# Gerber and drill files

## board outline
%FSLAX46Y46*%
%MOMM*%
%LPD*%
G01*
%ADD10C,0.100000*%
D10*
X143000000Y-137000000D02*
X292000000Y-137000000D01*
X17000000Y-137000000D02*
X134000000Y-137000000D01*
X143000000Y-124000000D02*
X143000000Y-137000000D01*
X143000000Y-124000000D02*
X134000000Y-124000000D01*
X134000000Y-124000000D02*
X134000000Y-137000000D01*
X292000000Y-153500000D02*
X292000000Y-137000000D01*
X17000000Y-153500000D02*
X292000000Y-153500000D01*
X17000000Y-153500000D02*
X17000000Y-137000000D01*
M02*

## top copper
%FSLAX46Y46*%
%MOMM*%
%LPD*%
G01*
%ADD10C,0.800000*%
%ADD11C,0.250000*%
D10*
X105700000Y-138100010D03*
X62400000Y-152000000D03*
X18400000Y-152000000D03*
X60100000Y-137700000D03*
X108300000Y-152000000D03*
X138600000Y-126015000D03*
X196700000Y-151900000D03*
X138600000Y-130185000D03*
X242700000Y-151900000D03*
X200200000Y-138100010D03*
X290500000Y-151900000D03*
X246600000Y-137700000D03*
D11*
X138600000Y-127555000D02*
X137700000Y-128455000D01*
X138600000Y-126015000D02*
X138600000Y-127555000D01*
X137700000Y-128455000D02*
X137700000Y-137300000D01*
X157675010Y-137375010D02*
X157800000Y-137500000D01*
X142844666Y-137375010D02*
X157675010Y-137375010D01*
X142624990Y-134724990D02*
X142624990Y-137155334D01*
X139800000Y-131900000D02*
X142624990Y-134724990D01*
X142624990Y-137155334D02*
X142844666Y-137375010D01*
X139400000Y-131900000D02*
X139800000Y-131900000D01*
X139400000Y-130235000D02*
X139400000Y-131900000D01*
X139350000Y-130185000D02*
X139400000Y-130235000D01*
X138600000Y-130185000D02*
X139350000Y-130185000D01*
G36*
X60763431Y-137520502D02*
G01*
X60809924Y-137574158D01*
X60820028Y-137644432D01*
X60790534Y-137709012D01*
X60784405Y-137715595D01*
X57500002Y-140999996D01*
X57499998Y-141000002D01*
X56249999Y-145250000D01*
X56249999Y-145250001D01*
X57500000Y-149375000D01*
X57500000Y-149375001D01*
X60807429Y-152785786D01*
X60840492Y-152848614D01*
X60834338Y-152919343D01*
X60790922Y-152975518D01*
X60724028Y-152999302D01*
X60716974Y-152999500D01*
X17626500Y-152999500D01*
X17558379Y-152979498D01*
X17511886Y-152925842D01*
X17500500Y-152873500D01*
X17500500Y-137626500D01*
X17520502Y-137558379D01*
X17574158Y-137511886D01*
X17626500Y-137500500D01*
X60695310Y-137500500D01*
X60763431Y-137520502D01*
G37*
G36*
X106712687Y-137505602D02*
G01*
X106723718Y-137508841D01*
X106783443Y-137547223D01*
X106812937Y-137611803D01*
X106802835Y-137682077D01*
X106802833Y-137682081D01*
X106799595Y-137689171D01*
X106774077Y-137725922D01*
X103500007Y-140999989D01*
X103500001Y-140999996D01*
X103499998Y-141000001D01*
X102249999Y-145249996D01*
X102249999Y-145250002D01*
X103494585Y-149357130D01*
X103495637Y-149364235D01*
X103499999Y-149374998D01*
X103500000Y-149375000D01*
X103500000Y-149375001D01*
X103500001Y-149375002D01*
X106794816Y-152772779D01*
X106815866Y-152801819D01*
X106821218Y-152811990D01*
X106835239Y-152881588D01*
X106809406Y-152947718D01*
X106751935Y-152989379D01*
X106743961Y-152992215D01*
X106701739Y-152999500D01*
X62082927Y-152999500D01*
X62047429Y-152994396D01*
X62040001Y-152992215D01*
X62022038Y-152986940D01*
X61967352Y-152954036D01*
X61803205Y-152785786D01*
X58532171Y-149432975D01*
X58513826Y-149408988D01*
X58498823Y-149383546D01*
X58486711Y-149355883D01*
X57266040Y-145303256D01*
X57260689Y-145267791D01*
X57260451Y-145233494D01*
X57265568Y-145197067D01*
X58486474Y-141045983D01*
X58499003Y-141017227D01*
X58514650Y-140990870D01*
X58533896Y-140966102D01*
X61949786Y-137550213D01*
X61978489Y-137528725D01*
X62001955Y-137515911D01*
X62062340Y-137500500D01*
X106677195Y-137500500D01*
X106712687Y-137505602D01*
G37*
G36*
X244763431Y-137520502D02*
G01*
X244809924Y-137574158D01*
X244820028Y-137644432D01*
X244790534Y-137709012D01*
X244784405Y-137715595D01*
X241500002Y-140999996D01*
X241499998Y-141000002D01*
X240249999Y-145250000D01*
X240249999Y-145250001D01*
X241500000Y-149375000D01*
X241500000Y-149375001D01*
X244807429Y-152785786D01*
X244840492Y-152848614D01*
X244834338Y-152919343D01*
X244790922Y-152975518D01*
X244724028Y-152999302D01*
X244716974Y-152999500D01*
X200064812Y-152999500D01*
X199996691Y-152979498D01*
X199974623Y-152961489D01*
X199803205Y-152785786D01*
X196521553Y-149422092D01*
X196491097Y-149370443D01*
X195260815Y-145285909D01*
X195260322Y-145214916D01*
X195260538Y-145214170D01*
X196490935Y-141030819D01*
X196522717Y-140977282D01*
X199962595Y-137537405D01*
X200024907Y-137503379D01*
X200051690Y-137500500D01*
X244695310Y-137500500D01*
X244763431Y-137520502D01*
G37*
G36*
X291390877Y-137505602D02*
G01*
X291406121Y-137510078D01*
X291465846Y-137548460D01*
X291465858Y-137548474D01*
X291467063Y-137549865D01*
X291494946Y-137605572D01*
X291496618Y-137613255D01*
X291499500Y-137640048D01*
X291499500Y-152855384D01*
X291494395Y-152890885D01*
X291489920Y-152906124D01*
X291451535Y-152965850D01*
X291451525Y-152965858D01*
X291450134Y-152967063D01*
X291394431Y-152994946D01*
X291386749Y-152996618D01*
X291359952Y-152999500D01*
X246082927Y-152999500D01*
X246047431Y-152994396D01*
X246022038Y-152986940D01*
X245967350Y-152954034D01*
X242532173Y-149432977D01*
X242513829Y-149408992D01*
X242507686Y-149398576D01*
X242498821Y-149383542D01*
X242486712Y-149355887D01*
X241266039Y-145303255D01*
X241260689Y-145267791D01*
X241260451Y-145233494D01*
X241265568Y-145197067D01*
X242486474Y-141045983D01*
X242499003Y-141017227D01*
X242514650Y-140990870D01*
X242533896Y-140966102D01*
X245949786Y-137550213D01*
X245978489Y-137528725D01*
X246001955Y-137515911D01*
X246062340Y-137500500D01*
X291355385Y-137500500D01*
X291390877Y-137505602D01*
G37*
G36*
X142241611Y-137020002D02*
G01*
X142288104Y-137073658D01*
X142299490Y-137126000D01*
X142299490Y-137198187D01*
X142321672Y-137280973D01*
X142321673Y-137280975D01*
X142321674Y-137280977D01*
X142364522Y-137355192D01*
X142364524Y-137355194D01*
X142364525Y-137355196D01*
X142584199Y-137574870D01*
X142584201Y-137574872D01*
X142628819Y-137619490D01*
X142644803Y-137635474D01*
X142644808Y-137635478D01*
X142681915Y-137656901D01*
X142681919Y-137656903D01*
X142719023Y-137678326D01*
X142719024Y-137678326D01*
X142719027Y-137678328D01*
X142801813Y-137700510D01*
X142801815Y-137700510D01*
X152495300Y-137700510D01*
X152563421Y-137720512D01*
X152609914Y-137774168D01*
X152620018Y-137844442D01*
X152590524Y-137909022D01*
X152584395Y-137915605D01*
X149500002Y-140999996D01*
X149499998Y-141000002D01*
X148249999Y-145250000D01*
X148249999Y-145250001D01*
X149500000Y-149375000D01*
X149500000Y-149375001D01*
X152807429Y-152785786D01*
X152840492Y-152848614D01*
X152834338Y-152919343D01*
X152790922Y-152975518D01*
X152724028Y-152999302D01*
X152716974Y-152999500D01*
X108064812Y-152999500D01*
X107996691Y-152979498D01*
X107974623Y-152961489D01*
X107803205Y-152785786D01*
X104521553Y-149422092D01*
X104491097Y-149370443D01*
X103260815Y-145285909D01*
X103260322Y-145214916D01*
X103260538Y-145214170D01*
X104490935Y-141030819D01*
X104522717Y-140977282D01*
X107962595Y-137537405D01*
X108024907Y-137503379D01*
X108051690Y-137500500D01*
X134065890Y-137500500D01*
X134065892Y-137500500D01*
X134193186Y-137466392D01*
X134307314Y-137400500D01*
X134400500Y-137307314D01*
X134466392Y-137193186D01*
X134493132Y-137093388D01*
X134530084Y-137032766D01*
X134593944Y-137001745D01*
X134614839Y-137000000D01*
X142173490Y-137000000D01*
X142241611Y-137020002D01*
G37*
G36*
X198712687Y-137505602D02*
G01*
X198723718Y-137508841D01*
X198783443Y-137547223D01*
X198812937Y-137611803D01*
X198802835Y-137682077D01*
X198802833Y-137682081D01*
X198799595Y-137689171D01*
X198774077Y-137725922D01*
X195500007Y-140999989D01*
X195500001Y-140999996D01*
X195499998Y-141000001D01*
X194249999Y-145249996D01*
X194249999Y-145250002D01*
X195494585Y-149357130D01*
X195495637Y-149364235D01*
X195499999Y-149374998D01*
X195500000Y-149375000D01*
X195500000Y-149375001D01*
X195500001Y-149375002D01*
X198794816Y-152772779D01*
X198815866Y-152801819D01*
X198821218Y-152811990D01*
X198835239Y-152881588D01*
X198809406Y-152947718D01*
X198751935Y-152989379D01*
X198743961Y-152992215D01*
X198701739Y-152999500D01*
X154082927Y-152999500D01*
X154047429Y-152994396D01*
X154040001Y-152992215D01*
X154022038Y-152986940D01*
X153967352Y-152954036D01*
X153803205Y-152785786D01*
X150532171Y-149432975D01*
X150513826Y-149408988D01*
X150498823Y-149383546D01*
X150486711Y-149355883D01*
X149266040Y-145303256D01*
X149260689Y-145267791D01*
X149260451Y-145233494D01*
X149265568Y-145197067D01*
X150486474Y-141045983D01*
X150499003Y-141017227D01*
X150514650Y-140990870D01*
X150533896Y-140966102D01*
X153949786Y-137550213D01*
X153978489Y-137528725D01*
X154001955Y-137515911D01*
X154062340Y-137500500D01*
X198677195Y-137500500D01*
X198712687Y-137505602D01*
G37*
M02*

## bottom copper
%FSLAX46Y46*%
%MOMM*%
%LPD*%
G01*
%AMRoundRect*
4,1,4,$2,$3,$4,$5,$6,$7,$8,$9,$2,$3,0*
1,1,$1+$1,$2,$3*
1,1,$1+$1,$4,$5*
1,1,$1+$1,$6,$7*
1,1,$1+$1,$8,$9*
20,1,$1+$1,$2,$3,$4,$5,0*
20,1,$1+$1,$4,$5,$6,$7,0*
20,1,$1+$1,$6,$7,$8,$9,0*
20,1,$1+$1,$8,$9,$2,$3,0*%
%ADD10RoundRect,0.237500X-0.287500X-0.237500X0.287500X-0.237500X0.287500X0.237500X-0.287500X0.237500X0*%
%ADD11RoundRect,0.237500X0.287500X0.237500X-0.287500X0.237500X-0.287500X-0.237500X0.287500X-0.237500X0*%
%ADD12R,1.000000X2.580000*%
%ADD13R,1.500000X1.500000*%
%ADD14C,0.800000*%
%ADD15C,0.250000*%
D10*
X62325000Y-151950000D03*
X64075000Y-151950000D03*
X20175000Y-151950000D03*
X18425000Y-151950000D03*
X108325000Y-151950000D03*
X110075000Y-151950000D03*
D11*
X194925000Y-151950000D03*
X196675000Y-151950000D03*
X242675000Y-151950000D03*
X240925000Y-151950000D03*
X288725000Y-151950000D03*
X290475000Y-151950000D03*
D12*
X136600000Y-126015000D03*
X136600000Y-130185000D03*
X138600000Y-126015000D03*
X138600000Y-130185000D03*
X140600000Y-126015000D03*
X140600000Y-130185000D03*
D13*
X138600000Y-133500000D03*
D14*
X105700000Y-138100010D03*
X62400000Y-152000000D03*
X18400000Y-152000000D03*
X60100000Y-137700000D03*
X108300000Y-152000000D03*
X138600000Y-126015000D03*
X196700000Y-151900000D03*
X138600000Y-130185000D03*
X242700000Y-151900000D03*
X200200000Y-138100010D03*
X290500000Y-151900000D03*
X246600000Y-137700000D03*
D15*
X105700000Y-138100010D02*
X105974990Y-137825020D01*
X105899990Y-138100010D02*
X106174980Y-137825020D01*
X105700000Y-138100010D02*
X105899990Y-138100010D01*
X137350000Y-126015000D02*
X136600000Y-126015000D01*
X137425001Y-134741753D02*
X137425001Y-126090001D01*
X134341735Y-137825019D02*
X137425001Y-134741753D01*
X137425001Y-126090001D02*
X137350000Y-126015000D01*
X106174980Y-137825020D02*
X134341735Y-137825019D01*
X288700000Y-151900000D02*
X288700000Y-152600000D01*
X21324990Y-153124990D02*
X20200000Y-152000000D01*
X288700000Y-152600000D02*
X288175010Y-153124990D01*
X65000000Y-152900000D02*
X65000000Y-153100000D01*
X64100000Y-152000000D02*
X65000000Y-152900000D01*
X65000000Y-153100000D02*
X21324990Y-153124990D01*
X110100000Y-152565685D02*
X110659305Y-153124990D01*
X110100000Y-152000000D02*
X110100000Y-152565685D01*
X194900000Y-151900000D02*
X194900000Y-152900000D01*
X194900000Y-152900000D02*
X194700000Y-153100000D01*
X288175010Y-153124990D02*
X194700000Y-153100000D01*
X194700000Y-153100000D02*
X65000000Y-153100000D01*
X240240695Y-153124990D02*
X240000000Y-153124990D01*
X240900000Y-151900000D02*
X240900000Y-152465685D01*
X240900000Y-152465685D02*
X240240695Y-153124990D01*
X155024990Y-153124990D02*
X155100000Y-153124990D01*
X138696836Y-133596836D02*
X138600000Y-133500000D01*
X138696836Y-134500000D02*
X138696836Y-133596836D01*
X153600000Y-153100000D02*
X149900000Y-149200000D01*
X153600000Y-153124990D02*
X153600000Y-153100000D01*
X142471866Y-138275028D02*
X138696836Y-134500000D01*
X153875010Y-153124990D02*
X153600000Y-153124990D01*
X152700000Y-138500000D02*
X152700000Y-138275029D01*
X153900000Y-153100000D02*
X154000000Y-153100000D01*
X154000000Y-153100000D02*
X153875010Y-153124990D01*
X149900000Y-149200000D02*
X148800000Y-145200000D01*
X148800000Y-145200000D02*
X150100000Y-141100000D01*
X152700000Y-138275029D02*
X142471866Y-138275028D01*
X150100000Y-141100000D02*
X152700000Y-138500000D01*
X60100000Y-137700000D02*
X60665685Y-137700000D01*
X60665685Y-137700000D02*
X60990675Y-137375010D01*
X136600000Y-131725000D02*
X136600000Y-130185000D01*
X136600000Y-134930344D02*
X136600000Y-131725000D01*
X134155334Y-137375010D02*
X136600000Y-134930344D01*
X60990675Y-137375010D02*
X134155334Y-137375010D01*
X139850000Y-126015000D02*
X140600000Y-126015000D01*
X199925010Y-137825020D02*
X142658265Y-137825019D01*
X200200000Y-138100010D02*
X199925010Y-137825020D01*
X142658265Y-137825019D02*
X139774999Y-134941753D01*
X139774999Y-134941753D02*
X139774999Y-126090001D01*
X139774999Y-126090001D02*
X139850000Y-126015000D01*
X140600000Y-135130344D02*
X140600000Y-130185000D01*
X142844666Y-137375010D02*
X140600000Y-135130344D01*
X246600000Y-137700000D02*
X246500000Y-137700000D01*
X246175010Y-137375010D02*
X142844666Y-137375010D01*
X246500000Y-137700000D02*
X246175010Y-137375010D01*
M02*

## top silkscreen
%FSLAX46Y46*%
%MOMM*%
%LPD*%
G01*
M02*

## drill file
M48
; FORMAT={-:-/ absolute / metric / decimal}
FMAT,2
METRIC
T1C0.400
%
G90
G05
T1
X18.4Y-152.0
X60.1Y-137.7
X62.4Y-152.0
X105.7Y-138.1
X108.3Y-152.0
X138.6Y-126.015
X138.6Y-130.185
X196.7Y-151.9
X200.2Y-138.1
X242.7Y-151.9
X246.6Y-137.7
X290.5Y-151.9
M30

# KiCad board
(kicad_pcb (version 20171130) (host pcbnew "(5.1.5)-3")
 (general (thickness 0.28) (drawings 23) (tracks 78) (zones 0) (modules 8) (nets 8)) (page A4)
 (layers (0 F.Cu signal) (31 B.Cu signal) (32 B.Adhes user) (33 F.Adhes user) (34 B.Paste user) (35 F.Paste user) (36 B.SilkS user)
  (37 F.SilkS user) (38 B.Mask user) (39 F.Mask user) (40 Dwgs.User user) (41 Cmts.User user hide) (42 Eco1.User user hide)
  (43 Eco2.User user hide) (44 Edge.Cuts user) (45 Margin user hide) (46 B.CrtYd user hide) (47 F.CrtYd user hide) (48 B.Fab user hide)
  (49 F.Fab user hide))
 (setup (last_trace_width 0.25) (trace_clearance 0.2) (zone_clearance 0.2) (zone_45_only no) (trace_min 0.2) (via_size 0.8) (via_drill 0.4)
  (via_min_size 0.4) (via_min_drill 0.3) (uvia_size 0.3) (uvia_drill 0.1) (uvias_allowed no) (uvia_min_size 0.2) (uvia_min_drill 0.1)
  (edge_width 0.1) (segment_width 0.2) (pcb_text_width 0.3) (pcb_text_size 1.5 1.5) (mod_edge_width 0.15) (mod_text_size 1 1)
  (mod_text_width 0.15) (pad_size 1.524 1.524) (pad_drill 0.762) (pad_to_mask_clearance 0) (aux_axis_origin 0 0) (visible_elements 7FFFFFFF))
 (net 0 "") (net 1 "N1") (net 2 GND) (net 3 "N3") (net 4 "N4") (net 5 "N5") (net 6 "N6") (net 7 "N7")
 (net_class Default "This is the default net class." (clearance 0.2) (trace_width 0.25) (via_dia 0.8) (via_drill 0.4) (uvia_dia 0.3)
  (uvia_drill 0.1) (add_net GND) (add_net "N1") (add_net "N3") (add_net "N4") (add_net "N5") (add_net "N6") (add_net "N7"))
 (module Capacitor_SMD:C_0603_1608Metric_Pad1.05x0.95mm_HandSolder (layer B.Cu) (at 63.2 151.95)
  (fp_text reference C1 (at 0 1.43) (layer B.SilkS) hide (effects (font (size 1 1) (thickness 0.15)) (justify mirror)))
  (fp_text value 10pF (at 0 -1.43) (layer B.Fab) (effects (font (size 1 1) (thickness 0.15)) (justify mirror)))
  (pad 1 smd roundrect (at -0.875 0) (size 1.05 0.95) (layers B.Cu B.Paste B.Mask) (roundrect_rratio 0.25) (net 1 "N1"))
  (pad 2 smd roundrect (at 0.875 0) (size 1.05 0.95) (layers B.Cu B.Paste B.Mask) (roundrect_rratio 0.25) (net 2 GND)))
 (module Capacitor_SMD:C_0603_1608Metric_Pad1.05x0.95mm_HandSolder (layer B.Cu) (at 19.3 151.95)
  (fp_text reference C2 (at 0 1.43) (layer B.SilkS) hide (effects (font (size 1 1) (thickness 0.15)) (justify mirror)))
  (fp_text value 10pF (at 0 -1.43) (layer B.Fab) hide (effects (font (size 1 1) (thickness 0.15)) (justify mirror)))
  (pad 2 smd roundrect (at 0.875 0) (size 1.05 0.95) (layers B.Cu B.Paste B.Mask) (roundrect_rratio 0.25) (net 2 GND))
  (pad 1 smd roundrect (at -0.875 0) (size 1.05 0.95) (layers B.Cu B.Paste B.Mask) (roundrect_rratio 0.25) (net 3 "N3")))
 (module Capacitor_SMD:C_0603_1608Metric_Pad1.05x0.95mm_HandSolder (layer B.Cu) (at 109.2 151.95)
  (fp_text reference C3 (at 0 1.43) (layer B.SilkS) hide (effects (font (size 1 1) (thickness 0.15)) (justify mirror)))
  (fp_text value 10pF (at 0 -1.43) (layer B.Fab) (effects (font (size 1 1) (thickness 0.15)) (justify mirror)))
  (pad 1 smd roundrect (at -0.875 0) (size 1.05 0.95) (layers B.Cu B.Paste B.Mask) (roundrect_rratio 0.25) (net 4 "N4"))
  (pad 2 smd roundrect (at 0.875 0) (size 1.05 0.95) (layers B.Cu B.Paste B.Mask) (roundrect_rratio 0.25) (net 2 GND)))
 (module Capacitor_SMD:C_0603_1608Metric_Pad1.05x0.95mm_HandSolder (layer B.Cu) (at 195.8 151.95 180)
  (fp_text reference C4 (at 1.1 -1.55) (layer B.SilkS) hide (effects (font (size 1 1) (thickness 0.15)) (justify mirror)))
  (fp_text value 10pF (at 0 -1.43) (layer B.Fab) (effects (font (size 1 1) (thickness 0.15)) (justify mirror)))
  (pad 2 smd roundrect (at 0.875 0 180) (size 1.05 0.95) (layers B.Cu B.Paste B.Mask) (roundrect_rratio 0.25) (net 2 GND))
  (pad 1 smd roundrect (at -0.875 0 180) (size 1.05 0.95) (layers B.Cu B.Paste B.Mask) (roundrect_rratio 0.25) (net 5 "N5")))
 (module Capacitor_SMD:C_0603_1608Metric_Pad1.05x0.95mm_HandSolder (layer B.Cu) (at 241.8 151.95 180)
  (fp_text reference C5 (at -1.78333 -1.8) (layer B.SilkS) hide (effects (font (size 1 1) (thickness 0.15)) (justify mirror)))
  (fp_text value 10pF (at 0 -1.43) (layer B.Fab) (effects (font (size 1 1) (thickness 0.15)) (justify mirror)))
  (pad 1 smd roundrect (at -0.875 0 180) (size 1.05 0.95) (layers B.Cu B.Paste B.Mask) (roundrect_rratio 0.25) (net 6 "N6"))
  (pad 2 smd roundrect (at 0.875 0 180) (size 1.05 0.95) (layers B.Cu B.Paste B.Mask) (roundrect_rratio 0.25) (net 2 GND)))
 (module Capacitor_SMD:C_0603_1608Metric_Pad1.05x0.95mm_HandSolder (layer B.Cu) (at 289.6 151.95 180)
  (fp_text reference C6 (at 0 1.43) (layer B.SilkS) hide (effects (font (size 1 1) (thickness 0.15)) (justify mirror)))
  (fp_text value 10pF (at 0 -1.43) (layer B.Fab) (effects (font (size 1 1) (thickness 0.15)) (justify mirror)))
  (pad 2 smd roundrect (at 0.875 0 180) (size 1.05 0.95) (layers B.Cu B.Paste B.Mask) (roundrect_rratio 0.25) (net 2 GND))
  (pad 1 smd roundrect (at -0.875 0 180) (size 1.05 0.95) (layers B.Cu B.Paste B.Mask) (roundrect_rratio 0.25) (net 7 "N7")))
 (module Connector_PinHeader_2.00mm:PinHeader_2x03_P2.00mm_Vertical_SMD (layer B.Cu) (at 138.6 128.1 270)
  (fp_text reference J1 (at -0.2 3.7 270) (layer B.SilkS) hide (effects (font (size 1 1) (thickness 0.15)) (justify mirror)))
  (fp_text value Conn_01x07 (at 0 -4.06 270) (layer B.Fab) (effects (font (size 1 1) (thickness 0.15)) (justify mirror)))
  (pad 1 smd rect (at -2.085 2 270) (size 2.58 1) (layers B.Cu B.Paste B.Mask) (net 1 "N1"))
  (pad 2 smd rect (at 2.085 2 270) (size 2.58 1) (layers B.Cu B.Paste B.Mask) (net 3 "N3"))
  (pad 3 smd rect (at -2.085 0 270) (size 2.58 1) (layers B.Cu B.Paste B.Mask) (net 4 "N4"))
  (pad 4 smd rect (at 2.085 0 270) (size 2.58 1) (layers B.Cu B.Paste B.Mask) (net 5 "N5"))
  (pad 5 smd rect (at -2.085 -2 270) (size 2.58 1) (layers B.Cu B.Paste B.Mask) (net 6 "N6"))
  (pad 6 smd rect (at 2.085 -2 270) (size 2.58 1) (layers B.Cu B.Paste B.Mask) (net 7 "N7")))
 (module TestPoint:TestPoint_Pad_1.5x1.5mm (layer B.Cu) (at 138.6 133.5)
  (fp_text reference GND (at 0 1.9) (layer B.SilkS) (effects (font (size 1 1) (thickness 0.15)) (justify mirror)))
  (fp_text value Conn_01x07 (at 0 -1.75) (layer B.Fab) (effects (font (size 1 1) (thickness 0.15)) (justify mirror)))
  (pad 1 smd rect (at 0 0) (size 1.5 1.5) (layers B.Cu B.Mask) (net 2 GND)))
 (gr_line (start 143 137) (end 292 137) (layer Edge.Cuts) (width 0.1))
 (gr_line (start 17 137) (end 134 137) (layer Edge.Cuts) (width 0.1))
 (gr_line (start 143 124) (end 143 137) (layer Edge.Cuts) (width 0.1))
 (gr_line (start 143 124) (end 134 124) (layer Edge.Cuts) (width 0.1))
 (gr_line (start 134 124) (end 134 137) (layer Edge.Cuts) (width 0.1))
 (gr_line (start 292 153.5) (end 292 137) (layer Edge.Cuts) (width 0.1))
 (gr_line (start 17 153.5) (end 292 153.5) (layer Edge.Cuts) (width 0.1))
 (gr_line (start 17 153.5) (end 17 137) (layer Edge.Cuts) (width 0.1))
 (via (at 105.7 138.10001) (size 0.8) (drill 0.4) (layers F.Cu B.Cu) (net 1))
 (via (at 62.4 152) (size 0.8) (drill 0.4) (layers F.Cu B.Cu) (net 1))
 (segment (start 105.7 138.10001) (end 105.97499 137.82502) (width 0.25) (layer B.Cu) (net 1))
 (segment (start 105.89999 138.10001) (end 106.17498 137.82502) (width 0.25) (layer B.Cu) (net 1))
 (segment (start 105.7 138.10001) (end 105.89999 138.10001) (width 0.25) (layer B.Cu) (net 1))
 (segment (start 137.35 126.015) (end 136.6 126.015) (width 0.25) (layer B.Cu) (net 1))
 (segment (start 137.425001 134.741753) (end 137.425001 126.090001) (width 0.25) (layer B.Cu) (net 1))
 (segment (start 134.341735 137.825019) (end 137.425001 134.741753) (width 0.25) (layer B.Cu) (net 1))
 (segment (start 137.425001 126.090001) (end 137.35 126.015) (width 0.25) (layer B.Cu) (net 1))
 (segment (start 106.17498 137.82502) (end 134.341735 137.825019) (width 0.25) (layer B.Cu) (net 1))
 (segment (start 288.7 151.9) (end 288.7 152.6) (width 0.25) (layer B.Cu) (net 2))
 (segment (start 21.32499 153.12499) (end 20.2 152) (width 0.25) (layer B.Cu) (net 2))
 (segment (start 288.7 152.6) (end 288.17501 153.12499) (width 0.25) (layer B.Cu) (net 2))
 (segment (start 65 152.9) (end 65 153.1) (width 0.25) (layer B.Cu) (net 2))
 (segment (start 64.1 152) (end 65 152.9) (width 0.25) (layer B.Cu) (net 2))
 (segment (start 65 153.1) (end 21.32499 153.12499) (width 0.25) (layer B.Cu) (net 2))
 (segment (start 110.1 152.565685) (end 110.659305 153.12499) (width 0.25) (layer B.Cu) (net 2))
 (segment (start 110.1 152) (end 110.1 152.565685) (width 0.25) (layer B.Cu) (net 2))
 (segment (start 194.9 151.9) (end 194.9 152.9) (width 0.25) (layer B.Cu) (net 2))
 (segment (start 194.9 152.9) (end 194.7 153.1) (width 0.25) (layer B.Cu) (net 2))
 (segment (start 288.17501 153.12499) (end 194.7 153.1) (width 0.25) (layer B.Cu) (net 2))
 (segment (start 194.7 153.1) (end 65 153.1) (width 0.25) (layer B.Cu) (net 2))
 (segment (start 240.240695 153.12499) (end 240 153.12499) (width 0.25) (layer B.Cu) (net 2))
 (segment (start 240.9 151.9) (end 240.9 152.465685) (width 0.25) (layer B.Cu) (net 2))
 (segment (start 240.9 152.465685) (end 240.240695 153.12499) (width 0.25) (layer B.Cu) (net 2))
 (segment (start 155.02499 153.12499) (end 155.1 153.12499) (width 0.25) (layer B.Cu) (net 2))
 (segment (start 138.696836 133.596836) (end 138.6 133.5) (width 0.25) (layer B.Cu) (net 2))
 (segment (start 138.696836 134.5) (end 138.696836 133.596836) (width 0.25) (layer B.Cu) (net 2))
 (segment (start 153.6 153.1) (end 149.9 149.2) (width 0.25) (layer B.Cu) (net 2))
 (segment (start 153.6 153.12499) (end 153.6 153.1) (width 0.25) (layer B.Cu) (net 2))
 (segment (start 142.471866 138.275028) (end 138.696836 134.5) (width 0.25) (layer B.Cu) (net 2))
 (segment (start 153.87501 153.12499) (end 153.6 153.12499) (width 0.25) (layer B.Cu) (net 2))
 (segment (start 152.7 138.5) (end 152.7 138.275029) (width 0.25) (layer B.Cu) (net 2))
 (segment (start 153.9 153.1) (end 154 153.1) (width 0.25) (layer B.Cu) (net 2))
 (segment (start 154 153.1) (end 153.87501 153.12499) (width 0.25) (layer B.Cu) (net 2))
 (segment (start 149.9 149.2) (end 148.8 145.2) (width 0.25) (layer B.Cu) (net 2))
 (segment (start 148.8 145.2) (end 150.1 141.1) (width 0.25) (layer B.Cu) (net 2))
 (segment (start 152.7 138.275029) (end 142.471866 138.275028) (width 0.25) (layer B.Cu) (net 2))
 (segment (start 150.1 141.1) (end 152.7 138.5) (width 0.25) (layer B.Cu) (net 2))
 (via (at 18.4 152) (size 0.8) (drill 0.4) (layers F.Cu B.Cu) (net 3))
 (via (at 60.1 137.7) (size 0.8) (drill 0.4) (layers F.Cu B.Cu) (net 3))
 (segment (start 60.1 137.7) (end 60.665685 137.7) (width 0.25) (layer B.Cu) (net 3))
 (segment (start 60.665685 137.7) (end 60.990675 137.37501) (width 0.25) (layer B.Cu) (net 3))
 (segment (start 136.6 131.725) (end 136.6 130.185) (width 0.25) (layer B.Cu) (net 3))
 (segment (start 136.6 134.930344) (end 136.6 131.725) (width 0.25) (layer B.Cu) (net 3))
 (segment (start 134.155334 137.37501) (end 136.6 134.930344) (width 0.25) (layer B.Cu) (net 3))
 (segment (start 60.990675 137.37501) (end 134.155334 137.37501) (width 0.25) (layer B.Cu) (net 3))
 (via (at 108.3 152) (size 0.8) (drill 0.4) (layers F.Cu B.Cu) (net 4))
 (via (at 138.6 126.015) (size 0.8) (drill 0.4) (layers F.Cu B.Cu) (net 4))
 (segment (start 138.6 127.555) (end 137.7 128.455) (width 0.25) (layer F.Cu) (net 4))
 (segment (start 138.6 126.015) (end 138.6 127.555) (width 0.25) (layer F.Cu) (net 4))
 (segment (start 137.7 128.455) (end 137.7 137.3) (width 0.25) (layer F.Cu) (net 4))
 (via (at 196.7 151.9) (size 0.8) (drill 0.4) (layers F.Cu B.Cu) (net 5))
 (via (at 138.6 130.185) (size 0.8) (drill 0.4) (layers F.Cu B.Cu) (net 5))
 (segment (start 157.67501 137.37501) (end 157.8 137.5) (width 0.25) (layer F.Cu) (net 5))
 (segment (start 142.844666 137.37501) (end 157.67501 137.37501) (width 0.25) (layer F.Cu) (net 5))
 (segment (start 142.62499 134.72499) (end 142.62499 137.155334) (width 0.25) (layer F.Cu) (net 5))
 (segment (start 139.8 131.9) (end 142.62499 134.72499) (width 0.25) (layer F.Cu) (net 5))
 (segment (start 142.62499 137.155334) (end 142.844666 137.37501) (width 0.25) (layer F.Cu) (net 5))
 (segment (start 139.4 131.9) (end 139.8 131.9) (width 0.25) (layer F.Cu) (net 5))
 (segment (start 139.4 130.235) (end 139.4 131.9) (width 0.25) (layer F.Cu) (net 5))
 (segment (start 139.35 130.185) (end 139.4 130.235) (width 0.25) (layer F.Cu) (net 5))
 (segment (start 138.6 130.185) (end 139.35 130.185) (width 0.25) (layer F.Cu) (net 5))
 (via (at 242.7 151.9) (size 0.8) (drill 0.4) (layers F.Cu B.Cu) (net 6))
 (via (at 200.2 138.10001) (size 0.8) (drill 0.4) (layers F.Cu B.Cu) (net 6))
 (segment (start 139.85 126.015) (end 140.6 126.015) (width 0.25) (layer B.Cu) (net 6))
 (segment (start 199.92501 137.82502) (end 142.658265 137.825019) (width 0.25) (layer B.Cu) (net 6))
 (segment (start 200.2 138.10001) (end 199.92501 137.82502) (width 0.25) (layer B.Cu) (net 6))
 (segment (start 142.658265 137.825019) (end 139.774999 134.941753) (width 0.25) (layer B.Cu) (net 6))
 (segment (start 139.774999 134.941753) (end 139.774999 126.090001) (width 0.25) (layer B.Cu) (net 6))
 (segment (start 139.774999 126.090001) (end 139.85 126.015) (width 0.25) (layer B.Cu) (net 6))
 (via (at 290.5 151.9) (size 0.8) (drill 0.4) (layers F.Cu B.Cu) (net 7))
 (via (at 246.6 137.7) (size 0.8) (drill 0.4) (layers F.Cu B.Cu) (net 7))
 (segment (start 140.6 135.130344) (end 140.6 130.185) (width 0.25) (layer B.Cu) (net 7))
 (segment (start 142.844666 137.37501) (end 140.6 135.130344) (width 0.25) (layer B.Cu) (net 7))
 (segment (start 246.6 137.7) (end 246.5 137.7) (width 0.25) (layer B.Cu) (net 7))
 (segment (start 246.17501 137.37501) (end 142.844666 137.37501) (width 0.25) (layer B.Cu) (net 7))
 (segment (start 246.5 137.7) (end 246.17501 137.37501) (width 0.25) (layer B.Cu) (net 7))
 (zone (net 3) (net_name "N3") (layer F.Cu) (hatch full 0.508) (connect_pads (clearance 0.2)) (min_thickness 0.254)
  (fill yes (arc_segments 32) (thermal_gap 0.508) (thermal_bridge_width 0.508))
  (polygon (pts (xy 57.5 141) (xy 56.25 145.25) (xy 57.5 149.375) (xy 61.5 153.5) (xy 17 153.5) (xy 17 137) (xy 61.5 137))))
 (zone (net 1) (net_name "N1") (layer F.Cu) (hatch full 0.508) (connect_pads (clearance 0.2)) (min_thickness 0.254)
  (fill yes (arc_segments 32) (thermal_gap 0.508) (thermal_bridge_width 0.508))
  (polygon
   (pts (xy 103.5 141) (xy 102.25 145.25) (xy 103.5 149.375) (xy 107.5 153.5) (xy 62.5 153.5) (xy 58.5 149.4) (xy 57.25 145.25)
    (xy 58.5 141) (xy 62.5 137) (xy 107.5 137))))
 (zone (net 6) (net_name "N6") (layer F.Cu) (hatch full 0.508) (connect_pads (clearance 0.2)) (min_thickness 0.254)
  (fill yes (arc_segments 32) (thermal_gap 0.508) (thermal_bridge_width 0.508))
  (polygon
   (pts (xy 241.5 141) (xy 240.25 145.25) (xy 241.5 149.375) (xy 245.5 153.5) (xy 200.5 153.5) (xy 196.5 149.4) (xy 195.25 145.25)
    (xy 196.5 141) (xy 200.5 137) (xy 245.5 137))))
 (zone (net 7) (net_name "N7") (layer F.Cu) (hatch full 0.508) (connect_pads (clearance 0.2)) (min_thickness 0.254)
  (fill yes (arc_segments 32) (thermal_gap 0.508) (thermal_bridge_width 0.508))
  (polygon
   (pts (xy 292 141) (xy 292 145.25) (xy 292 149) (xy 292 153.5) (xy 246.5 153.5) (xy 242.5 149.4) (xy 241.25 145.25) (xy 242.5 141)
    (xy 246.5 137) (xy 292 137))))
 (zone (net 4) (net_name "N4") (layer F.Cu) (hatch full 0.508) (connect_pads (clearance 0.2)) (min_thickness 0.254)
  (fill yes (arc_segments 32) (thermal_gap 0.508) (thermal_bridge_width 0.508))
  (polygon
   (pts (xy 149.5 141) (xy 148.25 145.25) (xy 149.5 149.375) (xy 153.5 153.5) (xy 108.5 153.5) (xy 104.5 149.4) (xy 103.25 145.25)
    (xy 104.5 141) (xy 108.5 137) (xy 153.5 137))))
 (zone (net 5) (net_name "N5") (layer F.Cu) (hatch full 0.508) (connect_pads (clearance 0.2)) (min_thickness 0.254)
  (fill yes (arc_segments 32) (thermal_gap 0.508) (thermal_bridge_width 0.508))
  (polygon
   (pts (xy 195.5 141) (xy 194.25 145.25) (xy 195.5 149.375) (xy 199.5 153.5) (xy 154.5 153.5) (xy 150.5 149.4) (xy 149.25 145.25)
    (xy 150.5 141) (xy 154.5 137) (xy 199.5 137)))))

